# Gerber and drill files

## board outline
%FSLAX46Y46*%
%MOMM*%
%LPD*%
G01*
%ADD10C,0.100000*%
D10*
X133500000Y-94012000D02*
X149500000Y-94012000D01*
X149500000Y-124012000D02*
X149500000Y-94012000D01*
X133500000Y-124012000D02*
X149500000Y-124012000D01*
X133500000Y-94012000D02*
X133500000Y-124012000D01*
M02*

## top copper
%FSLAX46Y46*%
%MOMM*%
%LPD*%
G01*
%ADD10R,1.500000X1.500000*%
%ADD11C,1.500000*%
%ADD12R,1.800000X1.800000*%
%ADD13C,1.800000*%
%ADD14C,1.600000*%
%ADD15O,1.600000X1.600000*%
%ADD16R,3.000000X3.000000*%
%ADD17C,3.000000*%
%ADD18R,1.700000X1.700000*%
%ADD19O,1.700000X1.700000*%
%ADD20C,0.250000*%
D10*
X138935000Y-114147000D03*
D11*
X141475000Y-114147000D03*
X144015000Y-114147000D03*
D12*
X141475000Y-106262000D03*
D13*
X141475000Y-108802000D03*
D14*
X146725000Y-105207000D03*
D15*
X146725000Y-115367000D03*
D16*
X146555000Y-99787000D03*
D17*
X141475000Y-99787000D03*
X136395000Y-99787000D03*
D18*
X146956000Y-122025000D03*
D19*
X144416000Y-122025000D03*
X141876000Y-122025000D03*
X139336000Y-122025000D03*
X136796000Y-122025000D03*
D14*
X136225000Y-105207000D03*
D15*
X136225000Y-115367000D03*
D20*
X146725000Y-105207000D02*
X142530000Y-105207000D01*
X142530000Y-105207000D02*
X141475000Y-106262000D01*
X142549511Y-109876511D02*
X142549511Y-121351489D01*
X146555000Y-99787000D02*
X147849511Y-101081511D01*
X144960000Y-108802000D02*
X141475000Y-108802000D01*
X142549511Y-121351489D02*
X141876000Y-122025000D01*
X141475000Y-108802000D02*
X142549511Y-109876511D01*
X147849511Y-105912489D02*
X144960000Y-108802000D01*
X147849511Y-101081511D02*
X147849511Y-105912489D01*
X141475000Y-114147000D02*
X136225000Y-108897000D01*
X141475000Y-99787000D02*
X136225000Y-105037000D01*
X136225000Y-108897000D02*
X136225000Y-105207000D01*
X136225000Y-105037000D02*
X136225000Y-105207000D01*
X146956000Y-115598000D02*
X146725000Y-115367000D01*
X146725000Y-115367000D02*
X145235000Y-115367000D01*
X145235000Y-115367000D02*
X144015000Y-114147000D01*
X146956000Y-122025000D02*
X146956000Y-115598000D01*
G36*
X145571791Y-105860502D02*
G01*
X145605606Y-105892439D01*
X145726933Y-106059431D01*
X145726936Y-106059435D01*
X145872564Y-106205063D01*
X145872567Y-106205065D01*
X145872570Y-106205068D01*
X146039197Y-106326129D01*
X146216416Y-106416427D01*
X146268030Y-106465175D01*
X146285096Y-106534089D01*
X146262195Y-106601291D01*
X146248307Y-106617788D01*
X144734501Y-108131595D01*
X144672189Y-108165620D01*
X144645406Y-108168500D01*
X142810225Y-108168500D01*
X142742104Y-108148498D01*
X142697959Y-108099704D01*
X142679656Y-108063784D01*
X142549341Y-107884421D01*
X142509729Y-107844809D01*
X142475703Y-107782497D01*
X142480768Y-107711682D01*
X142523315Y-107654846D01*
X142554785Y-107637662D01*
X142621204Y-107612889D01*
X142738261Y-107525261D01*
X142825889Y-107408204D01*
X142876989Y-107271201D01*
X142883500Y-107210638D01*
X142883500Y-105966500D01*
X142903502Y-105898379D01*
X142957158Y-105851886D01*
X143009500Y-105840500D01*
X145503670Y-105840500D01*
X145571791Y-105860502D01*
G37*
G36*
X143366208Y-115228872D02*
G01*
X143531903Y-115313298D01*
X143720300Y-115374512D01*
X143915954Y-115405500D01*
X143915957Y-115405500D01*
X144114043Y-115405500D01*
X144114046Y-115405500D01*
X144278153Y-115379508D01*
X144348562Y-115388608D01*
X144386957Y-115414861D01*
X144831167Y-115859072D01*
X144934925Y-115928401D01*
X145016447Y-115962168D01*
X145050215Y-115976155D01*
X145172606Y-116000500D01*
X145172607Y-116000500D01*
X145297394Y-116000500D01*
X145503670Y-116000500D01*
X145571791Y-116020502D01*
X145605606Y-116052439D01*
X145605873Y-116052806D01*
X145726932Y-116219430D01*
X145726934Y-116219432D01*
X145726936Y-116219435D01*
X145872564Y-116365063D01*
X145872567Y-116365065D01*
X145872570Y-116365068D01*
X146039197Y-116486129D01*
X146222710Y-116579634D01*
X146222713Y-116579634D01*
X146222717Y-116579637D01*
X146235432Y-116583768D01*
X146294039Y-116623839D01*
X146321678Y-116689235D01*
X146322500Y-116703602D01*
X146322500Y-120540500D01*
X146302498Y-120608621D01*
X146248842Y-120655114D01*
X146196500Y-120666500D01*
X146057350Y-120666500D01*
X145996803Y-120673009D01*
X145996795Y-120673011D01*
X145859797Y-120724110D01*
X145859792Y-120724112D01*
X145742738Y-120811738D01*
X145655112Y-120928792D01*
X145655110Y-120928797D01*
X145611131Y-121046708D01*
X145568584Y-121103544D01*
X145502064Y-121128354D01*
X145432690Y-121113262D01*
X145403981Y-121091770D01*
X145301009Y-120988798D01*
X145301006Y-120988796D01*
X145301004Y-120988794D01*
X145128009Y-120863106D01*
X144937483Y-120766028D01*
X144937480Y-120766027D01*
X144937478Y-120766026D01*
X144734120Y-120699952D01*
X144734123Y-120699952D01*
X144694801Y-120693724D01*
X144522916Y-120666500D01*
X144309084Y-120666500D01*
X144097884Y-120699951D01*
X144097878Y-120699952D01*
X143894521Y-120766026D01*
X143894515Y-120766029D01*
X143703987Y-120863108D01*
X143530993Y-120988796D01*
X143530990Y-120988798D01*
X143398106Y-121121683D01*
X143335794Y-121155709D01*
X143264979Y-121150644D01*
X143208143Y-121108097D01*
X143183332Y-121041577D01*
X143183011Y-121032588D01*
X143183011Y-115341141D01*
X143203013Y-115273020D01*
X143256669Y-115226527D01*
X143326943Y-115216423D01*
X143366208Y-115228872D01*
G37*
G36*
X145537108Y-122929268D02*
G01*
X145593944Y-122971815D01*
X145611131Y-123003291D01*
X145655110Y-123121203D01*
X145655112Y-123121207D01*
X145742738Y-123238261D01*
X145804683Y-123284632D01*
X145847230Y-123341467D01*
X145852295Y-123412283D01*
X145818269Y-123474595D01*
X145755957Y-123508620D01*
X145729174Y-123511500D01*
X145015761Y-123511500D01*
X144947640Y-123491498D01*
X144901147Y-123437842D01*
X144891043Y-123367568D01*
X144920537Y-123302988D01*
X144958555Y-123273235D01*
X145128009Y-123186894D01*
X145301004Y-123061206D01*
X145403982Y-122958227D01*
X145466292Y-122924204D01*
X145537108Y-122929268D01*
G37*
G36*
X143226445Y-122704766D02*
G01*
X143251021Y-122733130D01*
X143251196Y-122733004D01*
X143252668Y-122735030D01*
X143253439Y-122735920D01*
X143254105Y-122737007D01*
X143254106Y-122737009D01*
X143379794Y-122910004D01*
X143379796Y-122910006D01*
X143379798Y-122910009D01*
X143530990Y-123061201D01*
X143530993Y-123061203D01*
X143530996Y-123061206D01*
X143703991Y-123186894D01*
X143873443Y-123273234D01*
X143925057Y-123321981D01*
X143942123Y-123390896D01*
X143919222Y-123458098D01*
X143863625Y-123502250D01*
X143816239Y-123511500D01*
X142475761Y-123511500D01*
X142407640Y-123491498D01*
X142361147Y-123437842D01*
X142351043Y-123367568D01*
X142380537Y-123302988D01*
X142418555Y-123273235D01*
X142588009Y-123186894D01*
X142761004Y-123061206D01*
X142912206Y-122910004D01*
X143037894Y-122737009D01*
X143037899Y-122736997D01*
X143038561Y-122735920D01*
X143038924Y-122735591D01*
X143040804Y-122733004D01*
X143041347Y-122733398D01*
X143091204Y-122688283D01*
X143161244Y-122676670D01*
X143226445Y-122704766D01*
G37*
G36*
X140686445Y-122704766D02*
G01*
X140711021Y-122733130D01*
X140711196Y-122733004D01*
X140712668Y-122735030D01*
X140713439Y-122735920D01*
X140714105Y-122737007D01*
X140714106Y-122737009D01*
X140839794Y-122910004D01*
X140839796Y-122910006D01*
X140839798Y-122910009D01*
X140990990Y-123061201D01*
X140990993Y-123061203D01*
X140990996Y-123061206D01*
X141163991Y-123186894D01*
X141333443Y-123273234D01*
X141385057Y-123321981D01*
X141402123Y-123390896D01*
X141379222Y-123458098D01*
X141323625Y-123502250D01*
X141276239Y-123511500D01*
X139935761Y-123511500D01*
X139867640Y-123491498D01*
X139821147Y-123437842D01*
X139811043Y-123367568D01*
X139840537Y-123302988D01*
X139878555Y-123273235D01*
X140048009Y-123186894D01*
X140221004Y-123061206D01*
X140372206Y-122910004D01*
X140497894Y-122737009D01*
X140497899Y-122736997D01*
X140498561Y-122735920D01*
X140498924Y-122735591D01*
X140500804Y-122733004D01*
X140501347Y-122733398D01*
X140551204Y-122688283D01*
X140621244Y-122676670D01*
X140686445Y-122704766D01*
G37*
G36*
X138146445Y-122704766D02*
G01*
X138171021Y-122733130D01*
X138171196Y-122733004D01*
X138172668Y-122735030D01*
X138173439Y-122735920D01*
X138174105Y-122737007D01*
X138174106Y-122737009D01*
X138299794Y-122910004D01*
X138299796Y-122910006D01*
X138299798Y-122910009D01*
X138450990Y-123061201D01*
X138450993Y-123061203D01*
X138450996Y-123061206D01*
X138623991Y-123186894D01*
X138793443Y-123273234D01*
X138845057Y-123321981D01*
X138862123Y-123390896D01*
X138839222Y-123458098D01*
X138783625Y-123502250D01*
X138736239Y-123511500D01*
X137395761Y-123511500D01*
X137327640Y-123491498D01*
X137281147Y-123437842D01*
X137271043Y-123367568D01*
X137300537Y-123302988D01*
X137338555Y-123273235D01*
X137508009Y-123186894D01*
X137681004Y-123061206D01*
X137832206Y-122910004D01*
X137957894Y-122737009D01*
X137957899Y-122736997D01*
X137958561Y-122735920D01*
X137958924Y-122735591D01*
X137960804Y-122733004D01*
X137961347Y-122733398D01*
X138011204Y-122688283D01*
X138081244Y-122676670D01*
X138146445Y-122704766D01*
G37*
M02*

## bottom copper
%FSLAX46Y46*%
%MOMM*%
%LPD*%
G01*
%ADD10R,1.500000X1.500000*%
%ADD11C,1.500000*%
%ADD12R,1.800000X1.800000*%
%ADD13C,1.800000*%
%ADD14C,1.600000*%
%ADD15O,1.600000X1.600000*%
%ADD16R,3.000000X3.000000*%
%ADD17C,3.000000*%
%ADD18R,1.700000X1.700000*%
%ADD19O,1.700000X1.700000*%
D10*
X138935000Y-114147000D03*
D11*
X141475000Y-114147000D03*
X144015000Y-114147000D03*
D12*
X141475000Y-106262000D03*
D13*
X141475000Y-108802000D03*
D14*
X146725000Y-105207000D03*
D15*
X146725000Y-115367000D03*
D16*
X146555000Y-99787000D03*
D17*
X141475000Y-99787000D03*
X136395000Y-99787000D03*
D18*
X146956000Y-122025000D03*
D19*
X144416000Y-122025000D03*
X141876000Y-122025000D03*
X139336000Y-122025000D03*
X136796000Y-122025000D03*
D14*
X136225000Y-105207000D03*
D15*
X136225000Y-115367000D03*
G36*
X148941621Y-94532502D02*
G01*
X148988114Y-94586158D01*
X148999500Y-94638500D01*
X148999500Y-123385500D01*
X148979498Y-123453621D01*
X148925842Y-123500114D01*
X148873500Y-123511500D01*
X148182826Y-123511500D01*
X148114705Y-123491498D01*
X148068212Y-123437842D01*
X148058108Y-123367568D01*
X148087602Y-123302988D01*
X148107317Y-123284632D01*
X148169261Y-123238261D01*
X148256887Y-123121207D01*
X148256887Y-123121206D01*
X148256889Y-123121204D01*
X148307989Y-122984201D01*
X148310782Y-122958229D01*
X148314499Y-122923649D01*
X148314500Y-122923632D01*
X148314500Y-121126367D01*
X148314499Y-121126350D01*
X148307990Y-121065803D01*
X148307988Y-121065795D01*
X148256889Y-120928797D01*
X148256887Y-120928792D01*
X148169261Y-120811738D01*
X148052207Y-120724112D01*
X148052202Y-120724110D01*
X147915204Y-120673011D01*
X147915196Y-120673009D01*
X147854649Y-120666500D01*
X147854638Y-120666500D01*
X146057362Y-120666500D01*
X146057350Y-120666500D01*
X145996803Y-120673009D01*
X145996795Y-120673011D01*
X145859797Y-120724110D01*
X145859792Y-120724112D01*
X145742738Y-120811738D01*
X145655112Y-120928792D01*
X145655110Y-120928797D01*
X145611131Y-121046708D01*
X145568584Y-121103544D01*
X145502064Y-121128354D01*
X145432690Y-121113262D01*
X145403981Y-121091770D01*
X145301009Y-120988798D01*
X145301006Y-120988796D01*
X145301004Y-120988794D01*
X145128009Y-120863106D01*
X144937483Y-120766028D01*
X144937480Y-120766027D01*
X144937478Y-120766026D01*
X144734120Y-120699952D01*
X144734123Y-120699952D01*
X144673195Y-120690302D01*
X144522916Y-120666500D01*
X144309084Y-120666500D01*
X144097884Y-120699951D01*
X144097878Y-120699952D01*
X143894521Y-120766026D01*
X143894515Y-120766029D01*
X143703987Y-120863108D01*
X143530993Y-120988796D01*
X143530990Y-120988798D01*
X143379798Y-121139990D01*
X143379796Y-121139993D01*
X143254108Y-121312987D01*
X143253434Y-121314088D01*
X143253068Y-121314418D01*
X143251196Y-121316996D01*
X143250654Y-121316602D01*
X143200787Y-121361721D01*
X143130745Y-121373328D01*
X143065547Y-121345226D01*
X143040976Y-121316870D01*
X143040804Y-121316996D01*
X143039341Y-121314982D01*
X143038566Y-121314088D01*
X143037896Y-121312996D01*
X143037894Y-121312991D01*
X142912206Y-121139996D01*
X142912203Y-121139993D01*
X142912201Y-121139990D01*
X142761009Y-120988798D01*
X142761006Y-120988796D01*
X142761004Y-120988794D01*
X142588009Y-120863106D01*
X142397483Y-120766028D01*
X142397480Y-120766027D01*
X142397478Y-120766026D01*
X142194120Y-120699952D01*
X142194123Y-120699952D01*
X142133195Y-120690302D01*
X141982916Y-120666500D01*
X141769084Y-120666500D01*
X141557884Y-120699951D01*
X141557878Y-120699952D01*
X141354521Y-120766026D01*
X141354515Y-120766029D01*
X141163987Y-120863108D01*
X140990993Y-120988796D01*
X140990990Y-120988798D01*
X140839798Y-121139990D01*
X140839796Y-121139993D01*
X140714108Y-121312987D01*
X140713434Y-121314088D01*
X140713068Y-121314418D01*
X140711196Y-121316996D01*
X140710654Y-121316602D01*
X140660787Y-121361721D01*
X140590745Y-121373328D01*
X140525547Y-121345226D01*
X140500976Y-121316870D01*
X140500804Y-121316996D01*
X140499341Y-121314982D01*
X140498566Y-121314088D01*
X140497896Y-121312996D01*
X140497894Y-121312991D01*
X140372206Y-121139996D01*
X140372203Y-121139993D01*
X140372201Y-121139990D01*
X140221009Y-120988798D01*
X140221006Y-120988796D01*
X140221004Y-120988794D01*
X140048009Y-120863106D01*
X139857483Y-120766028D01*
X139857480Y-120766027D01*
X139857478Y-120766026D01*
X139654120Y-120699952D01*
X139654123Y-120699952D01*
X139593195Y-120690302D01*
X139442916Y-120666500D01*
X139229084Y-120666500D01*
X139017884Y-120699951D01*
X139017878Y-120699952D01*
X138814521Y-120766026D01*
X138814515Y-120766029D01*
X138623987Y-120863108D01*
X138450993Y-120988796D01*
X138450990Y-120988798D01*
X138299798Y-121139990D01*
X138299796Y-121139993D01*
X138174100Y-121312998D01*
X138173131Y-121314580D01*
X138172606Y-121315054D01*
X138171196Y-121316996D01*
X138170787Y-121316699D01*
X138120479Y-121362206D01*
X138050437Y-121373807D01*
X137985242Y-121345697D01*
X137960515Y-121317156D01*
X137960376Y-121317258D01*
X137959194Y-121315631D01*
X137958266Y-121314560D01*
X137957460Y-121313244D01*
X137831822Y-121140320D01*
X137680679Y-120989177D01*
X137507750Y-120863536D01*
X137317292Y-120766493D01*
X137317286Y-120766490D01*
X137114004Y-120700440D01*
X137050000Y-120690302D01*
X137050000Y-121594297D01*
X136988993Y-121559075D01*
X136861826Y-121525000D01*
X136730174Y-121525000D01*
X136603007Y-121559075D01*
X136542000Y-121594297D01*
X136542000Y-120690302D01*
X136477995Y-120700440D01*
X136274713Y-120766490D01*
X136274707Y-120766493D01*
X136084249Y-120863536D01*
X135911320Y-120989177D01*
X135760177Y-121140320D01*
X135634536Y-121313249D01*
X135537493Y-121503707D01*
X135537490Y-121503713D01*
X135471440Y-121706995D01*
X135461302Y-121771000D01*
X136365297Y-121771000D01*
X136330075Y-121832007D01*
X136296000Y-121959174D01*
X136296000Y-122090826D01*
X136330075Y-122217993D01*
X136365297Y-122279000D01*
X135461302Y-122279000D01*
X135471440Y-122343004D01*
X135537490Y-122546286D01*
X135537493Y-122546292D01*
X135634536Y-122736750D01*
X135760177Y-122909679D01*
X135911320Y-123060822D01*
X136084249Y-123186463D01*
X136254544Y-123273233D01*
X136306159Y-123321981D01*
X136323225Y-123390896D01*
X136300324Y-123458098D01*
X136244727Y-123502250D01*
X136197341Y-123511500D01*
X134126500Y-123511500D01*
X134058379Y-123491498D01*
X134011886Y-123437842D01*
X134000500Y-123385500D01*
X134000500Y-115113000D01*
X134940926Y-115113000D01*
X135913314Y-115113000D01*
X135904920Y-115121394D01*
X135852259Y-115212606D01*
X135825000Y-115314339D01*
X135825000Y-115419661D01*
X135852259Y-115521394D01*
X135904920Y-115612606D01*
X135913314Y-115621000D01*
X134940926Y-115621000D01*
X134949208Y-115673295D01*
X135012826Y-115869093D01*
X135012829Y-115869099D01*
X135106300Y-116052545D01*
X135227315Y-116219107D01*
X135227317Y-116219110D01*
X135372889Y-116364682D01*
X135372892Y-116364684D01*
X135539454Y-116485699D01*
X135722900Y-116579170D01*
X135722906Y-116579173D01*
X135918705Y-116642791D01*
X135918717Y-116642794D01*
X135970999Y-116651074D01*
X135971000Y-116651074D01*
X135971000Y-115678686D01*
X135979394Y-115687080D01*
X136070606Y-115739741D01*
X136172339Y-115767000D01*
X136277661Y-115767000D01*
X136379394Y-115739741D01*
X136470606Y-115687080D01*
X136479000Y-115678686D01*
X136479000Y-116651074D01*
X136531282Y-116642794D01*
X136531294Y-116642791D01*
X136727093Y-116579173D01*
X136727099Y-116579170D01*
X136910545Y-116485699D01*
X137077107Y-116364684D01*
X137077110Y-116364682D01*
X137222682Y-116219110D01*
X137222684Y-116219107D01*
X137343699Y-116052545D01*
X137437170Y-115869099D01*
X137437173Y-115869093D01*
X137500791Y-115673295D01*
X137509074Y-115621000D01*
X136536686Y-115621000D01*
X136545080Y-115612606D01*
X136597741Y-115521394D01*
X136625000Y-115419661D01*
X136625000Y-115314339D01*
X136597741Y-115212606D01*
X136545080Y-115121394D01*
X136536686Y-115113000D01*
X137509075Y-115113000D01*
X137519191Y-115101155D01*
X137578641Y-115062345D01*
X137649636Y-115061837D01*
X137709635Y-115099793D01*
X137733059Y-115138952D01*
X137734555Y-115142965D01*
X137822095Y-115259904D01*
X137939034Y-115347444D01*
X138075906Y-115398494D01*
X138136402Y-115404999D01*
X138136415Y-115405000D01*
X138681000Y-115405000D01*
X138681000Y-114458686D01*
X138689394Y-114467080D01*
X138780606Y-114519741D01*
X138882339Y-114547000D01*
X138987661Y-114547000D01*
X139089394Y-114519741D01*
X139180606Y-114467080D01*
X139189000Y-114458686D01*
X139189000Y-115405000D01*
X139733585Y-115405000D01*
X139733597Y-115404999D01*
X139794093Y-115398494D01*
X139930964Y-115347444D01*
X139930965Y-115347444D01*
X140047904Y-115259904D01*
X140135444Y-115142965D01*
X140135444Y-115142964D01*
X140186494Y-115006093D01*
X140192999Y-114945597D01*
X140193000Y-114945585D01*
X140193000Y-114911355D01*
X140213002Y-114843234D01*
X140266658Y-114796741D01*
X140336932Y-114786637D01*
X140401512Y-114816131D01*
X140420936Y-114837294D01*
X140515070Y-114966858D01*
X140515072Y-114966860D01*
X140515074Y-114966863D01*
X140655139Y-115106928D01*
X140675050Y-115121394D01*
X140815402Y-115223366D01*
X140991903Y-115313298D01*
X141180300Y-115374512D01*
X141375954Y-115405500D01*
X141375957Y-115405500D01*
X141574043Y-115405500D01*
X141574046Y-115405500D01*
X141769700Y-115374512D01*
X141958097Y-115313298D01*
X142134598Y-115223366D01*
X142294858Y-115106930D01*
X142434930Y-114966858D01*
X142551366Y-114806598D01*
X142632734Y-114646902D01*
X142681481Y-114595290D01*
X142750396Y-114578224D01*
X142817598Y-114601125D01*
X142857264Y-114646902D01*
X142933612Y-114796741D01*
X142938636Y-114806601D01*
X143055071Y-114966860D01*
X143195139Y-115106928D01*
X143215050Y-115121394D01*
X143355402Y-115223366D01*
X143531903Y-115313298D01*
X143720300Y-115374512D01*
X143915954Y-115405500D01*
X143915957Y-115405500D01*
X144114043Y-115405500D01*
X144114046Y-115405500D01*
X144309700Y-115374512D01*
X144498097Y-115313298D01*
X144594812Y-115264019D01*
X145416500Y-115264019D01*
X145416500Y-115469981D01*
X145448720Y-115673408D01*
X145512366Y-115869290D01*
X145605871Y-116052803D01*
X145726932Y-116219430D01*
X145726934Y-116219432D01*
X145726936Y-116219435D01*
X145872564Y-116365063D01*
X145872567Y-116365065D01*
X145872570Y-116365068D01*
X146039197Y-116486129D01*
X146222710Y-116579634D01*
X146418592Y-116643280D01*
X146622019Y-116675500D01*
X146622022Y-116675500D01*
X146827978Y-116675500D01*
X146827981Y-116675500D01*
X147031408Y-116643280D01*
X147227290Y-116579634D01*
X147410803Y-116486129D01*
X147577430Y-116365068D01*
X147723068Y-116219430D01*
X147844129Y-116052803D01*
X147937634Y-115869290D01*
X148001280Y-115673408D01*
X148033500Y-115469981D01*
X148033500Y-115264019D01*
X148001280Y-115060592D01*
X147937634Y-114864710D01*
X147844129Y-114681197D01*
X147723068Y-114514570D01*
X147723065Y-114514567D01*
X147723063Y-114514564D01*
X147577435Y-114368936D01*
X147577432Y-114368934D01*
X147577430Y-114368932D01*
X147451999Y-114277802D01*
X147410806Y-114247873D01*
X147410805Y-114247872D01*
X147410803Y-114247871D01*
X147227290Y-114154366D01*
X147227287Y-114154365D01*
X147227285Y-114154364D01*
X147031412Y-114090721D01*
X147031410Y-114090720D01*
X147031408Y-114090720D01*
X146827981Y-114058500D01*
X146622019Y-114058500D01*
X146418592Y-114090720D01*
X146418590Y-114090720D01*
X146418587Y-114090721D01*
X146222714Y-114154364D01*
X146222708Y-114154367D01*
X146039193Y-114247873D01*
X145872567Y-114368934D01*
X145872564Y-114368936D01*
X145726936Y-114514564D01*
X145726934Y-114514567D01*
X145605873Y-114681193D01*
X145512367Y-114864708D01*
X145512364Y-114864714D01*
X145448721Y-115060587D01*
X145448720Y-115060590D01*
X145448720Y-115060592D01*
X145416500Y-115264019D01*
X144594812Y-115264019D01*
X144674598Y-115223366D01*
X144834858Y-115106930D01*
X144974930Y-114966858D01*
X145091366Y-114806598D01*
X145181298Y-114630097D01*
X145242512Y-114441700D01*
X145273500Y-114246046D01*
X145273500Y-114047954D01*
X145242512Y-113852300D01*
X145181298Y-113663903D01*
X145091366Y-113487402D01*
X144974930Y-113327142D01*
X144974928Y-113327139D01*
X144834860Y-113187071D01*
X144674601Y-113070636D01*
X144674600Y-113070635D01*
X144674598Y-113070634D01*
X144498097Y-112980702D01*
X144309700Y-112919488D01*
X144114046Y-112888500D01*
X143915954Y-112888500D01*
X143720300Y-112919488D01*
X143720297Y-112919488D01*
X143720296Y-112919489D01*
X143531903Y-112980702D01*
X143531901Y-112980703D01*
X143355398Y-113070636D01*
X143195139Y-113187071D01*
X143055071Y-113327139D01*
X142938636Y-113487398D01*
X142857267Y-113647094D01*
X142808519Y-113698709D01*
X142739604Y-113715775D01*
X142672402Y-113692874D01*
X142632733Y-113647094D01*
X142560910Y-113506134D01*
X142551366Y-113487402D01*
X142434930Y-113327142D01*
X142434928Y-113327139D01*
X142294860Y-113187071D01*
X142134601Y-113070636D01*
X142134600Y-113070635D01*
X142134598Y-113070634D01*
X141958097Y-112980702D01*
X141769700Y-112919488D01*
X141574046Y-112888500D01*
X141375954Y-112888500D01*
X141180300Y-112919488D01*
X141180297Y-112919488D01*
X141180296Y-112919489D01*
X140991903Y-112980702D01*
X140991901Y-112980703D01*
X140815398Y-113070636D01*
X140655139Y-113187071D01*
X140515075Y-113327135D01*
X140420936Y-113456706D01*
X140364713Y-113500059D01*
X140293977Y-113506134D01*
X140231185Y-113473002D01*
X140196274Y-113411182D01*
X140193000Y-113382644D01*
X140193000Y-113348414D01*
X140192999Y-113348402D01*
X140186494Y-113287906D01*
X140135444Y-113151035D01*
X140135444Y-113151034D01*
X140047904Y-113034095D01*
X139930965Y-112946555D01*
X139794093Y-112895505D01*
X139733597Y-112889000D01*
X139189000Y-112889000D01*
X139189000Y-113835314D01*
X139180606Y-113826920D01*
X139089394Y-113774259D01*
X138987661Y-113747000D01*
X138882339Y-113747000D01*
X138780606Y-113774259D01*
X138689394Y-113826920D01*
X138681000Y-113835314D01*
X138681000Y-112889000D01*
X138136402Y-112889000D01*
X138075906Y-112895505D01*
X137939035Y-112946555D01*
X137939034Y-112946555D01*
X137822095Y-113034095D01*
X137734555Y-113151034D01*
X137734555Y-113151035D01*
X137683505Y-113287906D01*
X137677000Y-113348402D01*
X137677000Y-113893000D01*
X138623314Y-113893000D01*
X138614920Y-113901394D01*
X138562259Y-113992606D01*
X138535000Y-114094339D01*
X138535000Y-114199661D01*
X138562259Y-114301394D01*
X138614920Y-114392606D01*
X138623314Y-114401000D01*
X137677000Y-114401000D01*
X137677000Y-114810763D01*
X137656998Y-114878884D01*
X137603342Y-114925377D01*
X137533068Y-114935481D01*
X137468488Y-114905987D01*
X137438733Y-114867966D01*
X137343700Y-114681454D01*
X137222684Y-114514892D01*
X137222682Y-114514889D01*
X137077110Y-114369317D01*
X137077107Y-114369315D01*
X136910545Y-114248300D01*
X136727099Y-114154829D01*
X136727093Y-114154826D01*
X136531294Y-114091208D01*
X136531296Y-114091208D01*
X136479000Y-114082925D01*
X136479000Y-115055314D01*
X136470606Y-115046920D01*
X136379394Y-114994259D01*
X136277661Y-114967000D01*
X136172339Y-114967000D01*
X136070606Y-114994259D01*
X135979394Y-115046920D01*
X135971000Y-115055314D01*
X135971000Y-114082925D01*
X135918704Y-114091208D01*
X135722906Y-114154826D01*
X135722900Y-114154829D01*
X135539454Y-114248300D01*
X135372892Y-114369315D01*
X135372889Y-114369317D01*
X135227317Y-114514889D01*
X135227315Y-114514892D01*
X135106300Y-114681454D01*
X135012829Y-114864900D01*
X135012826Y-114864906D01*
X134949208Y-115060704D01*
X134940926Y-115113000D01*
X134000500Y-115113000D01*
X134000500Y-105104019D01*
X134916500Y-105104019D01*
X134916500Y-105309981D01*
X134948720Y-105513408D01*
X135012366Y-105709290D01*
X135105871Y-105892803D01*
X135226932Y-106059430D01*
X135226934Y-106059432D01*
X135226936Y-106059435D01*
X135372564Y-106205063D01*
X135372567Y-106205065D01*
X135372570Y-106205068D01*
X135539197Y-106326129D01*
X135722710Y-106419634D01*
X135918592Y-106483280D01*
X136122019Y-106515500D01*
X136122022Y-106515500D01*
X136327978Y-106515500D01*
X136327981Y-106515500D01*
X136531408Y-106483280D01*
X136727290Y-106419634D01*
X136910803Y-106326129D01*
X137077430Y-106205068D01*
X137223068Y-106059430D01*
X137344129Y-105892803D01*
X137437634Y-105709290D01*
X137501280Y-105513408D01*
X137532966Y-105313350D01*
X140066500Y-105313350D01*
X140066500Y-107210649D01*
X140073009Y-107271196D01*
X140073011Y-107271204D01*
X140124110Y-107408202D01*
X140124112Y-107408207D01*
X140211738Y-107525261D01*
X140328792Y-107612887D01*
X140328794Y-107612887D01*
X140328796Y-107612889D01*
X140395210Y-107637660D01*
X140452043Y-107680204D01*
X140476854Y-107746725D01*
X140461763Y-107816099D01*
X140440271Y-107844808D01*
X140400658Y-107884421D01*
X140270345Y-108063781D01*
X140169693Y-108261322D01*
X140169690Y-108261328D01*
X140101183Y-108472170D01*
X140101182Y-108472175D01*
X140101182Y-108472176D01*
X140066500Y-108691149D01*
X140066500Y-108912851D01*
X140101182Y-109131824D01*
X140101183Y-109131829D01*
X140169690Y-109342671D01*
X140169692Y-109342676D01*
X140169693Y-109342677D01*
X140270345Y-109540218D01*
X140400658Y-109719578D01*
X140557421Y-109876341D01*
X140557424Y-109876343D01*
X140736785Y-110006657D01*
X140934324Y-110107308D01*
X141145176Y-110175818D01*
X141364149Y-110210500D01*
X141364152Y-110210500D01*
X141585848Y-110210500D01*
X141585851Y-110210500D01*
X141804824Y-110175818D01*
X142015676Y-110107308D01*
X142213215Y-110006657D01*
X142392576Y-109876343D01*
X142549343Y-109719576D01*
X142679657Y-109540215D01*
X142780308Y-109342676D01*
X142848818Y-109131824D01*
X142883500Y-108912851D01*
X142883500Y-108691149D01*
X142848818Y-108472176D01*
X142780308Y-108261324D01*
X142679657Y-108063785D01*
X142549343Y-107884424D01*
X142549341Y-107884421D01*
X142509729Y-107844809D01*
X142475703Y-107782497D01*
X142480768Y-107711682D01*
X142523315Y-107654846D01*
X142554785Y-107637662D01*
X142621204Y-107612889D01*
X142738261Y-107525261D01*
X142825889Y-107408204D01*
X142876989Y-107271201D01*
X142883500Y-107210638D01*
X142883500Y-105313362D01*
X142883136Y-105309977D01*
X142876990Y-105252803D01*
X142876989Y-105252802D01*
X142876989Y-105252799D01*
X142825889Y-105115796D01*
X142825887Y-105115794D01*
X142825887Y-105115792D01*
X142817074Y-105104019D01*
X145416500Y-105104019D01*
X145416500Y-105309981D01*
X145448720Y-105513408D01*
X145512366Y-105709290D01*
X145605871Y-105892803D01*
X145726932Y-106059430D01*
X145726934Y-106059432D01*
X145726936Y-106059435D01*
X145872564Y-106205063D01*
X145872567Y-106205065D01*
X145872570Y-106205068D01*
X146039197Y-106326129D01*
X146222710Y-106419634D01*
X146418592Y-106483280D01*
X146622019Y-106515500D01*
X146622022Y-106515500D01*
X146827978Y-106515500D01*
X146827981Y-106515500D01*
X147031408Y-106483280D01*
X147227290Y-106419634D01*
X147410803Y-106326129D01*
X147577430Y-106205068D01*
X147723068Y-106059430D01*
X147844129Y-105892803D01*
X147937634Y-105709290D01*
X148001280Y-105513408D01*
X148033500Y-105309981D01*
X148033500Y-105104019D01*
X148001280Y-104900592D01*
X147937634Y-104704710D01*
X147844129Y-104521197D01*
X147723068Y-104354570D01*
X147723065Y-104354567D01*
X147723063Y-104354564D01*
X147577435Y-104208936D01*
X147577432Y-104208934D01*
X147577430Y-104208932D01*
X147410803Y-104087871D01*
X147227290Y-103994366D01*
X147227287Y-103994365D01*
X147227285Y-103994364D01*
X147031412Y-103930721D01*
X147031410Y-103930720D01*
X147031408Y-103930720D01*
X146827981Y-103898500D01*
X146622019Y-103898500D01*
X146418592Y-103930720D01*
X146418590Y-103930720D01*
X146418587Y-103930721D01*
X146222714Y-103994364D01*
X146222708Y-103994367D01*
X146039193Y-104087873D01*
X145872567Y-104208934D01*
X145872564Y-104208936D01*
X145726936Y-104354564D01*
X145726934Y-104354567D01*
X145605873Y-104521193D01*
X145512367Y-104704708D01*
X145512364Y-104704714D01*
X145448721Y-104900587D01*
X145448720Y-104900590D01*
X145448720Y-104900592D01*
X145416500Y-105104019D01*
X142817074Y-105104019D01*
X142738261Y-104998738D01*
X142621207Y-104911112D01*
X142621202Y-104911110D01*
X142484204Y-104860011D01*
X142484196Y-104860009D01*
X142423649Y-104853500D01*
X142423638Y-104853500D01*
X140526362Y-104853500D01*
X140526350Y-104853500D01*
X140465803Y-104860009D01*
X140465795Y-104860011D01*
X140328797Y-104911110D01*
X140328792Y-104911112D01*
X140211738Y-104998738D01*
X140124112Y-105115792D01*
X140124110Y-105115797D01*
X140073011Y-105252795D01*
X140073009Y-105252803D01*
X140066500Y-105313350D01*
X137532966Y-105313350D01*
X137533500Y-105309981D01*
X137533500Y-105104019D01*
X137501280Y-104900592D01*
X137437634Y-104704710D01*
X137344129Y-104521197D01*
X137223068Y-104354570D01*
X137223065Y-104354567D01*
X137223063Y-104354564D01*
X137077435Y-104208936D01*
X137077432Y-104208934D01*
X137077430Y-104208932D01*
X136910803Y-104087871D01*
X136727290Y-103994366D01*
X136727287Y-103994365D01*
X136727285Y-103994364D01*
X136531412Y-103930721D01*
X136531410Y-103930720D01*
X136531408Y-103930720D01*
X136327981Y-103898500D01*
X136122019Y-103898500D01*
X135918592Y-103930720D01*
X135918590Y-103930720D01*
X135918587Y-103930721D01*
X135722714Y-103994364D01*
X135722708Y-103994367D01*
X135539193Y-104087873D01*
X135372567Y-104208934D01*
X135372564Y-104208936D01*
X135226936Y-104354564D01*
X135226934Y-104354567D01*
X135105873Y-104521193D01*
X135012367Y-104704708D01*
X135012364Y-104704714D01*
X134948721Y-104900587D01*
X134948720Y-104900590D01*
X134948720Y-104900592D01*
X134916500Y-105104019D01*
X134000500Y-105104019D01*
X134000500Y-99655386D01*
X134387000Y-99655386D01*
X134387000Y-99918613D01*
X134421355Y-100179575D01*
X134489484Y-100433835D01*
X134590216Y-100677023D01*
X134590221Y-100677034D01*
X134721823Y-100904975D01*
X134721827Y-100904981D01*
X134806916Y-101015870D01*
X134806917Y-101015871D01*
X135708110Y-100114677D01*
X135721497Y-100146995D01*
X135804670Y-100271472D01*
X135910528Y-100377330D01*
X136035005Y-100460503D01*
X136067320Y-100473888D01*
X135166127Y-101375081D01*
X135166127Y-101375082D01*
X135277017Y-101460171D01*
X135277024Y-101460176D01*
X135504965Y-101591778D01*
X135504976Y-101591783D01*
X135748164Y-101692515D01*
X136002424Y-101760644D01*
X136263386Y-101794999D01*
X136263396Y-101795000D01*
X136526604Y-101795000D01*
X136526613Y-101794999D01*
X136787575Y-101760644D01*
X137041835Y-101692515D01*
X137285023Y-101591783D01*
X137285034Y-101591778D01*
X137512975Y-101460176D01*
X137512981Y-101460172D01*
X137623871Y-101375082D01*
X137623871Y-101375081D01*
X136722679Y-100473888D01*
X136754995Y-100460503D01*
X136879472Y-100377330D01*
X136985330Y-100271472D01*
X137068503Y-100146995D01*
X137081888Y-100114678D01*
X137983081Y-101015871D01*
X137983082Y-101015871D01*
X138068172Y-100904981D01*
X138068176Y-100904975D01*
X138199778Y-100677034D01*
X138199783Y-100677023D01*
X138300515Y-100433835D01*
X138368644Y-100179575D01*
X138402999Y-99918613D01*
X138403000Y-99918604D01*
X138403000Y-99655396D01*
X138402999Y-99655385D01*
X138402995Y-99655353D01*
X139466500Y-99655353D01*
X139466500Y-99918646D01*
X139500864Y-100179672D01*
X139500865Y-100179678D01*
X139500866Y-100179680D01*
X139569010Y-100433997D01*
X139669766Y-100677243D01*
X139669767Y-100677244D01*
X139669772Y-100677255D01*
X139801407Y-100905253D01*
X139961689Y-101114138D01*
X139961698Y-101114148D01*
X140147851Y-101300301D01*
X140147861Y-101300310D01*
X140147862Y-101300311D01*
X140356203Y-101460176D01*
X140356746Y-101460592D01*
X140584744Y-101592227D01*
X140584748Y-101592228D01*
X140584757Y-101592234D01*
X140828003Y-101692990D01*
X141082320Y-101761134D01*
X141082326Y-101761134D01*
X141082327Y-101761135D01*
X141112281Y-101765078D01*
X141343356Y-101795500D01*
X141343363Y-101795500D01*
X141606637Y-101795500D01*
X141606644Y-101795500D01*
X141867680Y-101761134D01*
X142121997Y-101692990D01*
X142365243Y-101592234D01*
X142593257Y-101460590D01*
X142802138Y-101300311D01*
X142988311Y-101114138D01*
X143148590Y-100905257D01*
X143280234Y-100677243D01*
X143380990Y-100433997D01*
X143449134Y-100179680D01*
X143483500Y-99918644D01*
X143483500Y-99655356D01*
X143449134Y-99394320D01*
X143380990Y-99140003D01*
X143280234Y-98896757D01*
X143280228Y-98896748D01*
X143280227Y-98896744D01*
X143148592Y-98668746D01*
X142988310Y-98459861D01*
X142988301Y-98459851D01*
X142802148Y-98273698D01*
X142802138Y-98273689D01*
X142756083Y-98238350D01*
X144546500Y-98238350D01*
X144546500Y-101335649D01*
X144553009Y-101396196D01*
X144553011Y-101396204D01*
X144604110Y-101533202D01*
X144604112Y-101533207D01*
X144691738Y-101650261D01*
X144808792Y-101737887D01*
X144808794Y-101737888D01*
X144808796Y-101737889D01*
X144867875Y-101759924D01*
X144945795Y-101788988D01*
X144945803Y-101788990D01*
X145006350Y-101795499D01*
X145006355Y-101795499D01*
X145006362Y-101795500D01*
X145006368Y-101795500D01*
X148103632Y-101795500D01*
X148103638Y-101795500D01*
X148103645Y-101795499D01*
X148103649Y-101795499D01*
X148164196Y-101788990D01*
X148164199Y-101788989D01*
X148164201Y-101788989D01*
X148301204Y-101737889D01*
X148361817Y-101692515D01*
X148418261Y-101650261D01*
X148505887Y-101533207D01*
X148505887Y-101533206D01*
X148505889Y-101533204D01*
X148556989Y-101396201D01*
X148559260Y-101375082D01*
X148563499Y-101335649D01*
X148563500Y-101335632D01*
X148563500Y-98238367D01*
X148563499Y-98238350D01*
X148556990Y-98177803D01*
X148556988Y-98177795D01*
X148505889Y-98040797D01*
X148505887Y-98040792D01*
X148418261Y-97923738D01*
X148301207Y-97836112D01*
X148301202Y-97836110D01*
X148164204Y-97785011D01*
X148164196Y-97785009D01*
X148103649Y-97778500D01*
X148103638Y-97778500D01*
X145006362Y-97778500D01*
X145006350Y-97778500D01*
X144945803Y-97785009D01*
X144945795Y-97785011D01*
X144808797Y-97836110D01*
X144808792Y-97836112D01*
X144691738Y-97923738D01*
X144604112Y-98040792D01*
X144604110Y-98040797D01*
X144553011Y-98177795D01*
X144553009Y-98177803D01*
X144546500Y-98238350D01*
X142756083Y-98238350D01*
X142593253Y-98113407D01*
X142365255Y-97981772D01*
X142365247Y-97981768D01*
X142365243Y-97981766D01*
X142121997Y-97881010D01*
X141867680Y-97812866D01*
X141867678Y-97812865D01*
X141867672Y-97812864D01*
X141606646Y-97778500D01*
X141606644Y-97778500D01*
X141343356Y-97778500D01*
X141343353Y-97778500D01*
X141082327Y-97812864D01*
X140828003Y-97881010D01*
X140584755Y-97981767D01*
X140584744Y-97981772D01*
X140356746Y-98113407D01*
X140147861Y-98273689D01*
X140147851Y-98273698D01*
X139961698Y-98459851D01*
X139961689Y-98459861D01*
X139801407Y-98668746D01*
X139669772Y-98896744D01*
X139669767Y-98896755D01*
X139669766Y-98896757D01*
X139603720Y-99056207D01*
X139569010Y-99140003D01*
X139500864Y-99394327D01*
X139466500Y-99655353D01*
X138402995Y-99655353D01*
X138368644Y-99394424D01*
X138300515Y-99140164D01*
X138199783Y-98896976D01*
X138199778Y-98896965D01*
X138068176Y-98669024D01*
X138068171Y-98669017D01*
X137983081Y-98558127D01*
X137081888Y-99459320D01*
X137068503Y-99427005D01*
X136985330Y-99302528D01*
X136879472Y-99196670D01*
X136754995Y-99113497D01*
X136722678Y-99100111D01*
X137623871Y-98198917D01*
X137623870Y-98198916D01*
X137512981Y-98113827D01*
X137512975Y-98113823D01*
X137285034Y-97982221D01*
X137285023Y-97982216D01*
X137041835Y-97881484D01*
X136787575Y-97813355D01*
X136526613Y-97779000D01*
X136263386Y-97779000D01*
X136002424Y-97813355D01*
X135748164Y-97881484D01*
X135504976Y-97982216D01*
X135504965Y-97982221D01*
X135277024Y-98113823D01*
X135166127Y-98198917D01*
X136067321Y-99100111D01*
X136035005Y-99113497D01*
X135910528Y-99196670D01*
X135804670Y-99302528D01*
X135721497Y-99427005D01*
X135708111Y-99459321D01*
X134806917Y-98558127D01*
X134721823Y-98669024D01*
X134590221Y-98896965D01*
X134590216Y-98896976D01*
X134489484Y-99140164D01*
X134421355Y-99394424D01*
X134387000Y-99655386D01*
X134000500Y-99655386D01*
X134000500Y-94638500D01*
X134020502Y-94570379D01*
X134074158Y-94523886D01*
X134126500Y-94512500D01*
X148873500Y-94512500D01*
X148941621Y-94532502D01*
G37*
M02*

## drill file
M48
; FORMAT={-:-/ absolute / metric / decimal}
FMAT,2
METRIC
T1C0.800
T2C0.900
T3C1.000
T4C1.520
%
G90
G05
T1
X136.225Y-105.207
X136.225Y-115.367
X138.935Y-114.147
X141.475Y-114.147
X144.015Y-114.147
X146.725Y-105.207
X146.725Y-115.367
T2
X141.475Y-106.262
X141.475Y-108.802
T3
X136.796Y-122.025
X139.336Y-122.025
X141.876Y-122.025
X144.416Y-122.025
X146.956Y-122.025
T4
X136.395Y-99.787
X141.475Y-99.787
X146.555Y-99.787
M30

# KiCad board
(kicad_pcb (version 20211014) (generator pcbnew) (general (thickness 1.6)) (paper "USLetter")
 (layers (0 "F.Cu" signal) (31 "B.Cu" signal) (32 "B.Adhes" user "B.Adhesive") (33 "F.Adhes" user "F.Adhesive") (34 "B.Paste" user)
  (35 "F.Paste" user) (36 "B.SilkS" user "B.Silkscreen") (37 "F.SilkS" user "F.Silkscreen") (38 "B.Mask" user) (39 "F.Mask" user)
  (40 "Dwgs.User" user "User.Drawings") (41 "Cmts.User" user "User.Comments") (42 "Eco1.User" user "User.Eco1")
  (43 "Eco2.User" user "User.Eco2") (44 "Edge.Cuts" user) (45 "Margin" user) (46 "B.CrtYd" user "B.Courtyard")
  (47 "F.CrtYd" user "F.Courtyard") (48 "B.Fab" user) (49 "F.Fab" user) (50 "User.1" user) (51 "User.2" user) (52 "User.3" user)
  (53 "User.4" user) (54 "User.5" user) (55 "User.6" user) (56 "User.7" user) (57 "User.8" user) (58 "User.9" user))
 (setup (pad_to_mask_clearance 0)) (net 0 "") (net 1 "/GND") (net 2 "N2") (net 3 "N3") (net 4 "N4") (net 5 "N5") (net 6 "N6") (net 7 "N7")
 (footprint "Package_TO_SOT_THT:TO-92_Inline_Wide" (layer "F.Cu") (at 138.935 114.147)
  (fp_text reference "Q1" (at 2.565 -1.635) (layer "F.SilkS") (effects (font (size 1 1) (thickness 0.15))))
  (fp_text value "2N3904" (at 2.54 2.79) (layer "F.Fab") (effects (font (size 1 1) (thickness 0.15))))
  (pad "1" thru_hole rect locked (at 0 0) (size 1.5 1.5) (drill 0.8) (layers *.Cu *.Mask) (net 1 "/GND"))
  (pad "2" thru_hole circle locked (at 2.54 0) (size 1.5 1.5) (drill 0.8) (layers *.Cu *.Mask) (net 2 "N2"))
  (pad "3" thru_hole circle locked (at 5.08 0) (size 1.5 1.5) (drill 0.8) (layers *.Cu *.Mask) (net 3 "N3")))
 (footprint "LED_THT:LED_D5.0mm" (layer "F.Cu") (at 141.475 106.262 -90)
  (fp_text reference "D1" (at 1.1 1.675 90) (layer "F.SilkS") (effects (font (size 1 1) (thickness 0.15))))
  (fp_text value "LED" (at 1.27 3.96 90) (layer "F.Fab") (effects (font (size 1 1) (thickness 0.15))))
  (pad "1" thru_hole rect locked (at 0 0 270) (size 1.8 1.8) (drill 0.9) (layers *.Cu *.Mask) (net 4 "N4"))
  (pad "2" thru_hole circle locked (at 2.54 0 270) (size 1.8 1.8) (drill 0.9) (layers *.Cu *.Mask) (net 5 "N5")))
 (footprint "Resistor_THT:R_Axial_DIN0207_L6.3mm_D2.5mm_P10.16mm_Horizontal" (layer "F.Cu") (at 146.725 105.207 -90)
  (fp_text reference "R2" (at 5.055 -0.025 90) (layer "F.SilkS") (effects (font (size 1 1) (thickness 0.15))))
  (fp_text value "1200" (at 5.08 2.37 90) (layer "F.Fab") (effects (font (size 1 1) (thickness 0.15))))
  (pad "1" thru_hole circle locked (at 0 0 270) (size 1.6 1.6) (drill 0.8) (layers *.Cu *.Mask) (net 4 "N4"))
  (pad "2" thru_hole oval locked (at 10.16 0 270) (size 1.6 1.6) (drill 0.8) (layers *.Cu *.Mask) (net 3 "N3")))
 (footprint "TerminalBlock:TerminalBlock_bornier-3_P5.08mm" (layer "F.Cu") (at 146.555 99.787 180)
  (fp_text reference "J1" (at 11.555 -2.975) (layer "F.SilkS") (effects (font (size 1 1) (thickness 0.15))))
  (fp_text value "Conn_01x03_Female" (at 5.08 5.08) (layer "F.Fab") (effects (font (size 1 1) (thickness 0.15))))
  (pad "1" thru_hole rect locked (at 0 0 180) (size 3 3) (drill 1.52) (layers *.Cu *.Mask) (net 5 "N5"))
  (pad "2" thru_hole circle locked (at 5.08 0 180) (size 3 3) (drill 1.52) (layers *.Cu *.Mask) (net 2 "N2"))
  (pad "3" thru_hole circle locked (at 10.16 0 180) (size 3 3) (drill 1.52) (layers *.Cu *.Mask) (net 1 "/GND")))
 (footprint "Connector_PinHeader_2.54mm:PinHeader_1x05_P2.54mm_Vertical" (layer "F.Cu") (at 146.956 122.025 -90)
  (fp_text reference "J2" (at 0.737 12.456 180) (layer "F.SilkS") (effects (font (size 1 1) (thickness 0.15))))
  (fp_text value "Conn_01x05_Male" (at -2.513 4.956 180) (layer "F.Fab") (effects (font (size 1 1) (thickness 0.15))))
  (pad "1" thru_hole rect locked (at 0 0 270) (size 1.7 1.7) (drill 1) (layers *.Cu *.Mask) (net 3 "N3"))
  (pad "2" thru_hole oval locked (at 0 2.54 270) (size 1.7 1.7) (drill 1) (layers *.Cu *.Mask) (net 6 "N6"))
  (pad "3" thru_hole oval locked (at 0 5.08 270) (size 1.7 1.7) (drill 1) (layers *.Cu *.Mask) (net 5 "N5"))
  (pad "4" thru_hole oval locked (at 0 7.62 270) (size 1.7 1.7) (drill 1) (layers *.Cu *.Mask) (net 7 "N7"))
  (pad "5" thru_hole oval locked (at 0 10.16 270) (size 1.7 1.7) (drill 1) (layers *.Cu *.Mask) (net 1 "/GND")))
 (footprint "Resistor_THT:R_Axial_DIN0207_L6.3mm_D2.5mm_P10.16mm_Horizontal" (layer "F.Cu") (at 136.225 105.207 -90)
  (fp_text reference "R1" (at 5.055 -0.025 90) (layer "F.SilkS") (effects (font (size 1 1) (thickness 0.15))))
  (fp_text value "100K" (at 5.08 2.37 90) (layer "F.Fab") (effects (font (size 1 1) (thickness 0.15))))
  (pad "1" thru_hole circle locked (at 0 0 270) (size 1.6 1.6) (drill 0.8) (layers *.Cu *.Mask) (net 2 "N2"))
  (pad "2" thru_hole oval locked (at 10.16 0 270) (size 1.6 1.6) (drill 0.8) (layers *.Cu *.Mask) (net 1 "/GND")))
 (gr_line (start 133.5 94.012) (end 149.5 94.012) (layer "Edge.Cuts") (width 0.1))
 (gr_line (start 149.5 124.012) (end 149.5 94.012) (layer "Edge.Cuts") (width 0.1))
 (gr_line (start 133.5 124.012) (end 149.5 124.012) (layer "Edge.Cuts") (width 0.1))
 (gr_line (start 133.5 94.012) (end 133.5 124.012) (layer "Edge.Cuts") (width 0.1))
 (segment (start 146.725 105.207) (end 142.53 105.207) (width 0.25) (layer "F.Cu") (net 4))
 (segment (start 142.53 105.207) (end 141.475 106.262) (width 0.25) (layer "F.Cu") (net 4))
 (segment (start 142.549511 109.876511) (end 142.549511 121.351489) (width 0.25) (layer "F.Cu") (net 5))
 (segment (start 146.555 99.787) (end 147.849511 101.081511) (width 0.25) (layer "F.Cu") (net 5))
 (segment (start 144.96 108.802) (end 141.475 108.802) (width 0.25) (layer "F.Cu") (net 5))
 (segment (start 142.549511 121.351489) (end 141.876 122.025) (width 0.25) (layer "F.Cu") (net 5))
 (segment (start 141.475 108.802) (end 142.549511 109.876511) (width 0.25) (layer "F.Cu") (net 5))
 (segment (start 147.849511 105.912489) (end 144.96 108.802) (width 0.25) (layer "F.Cu") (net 5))
 (segment (start 147.849511 101.081511) (end 147.849511 105.912489) (width 0.25) (layer "F.Cu") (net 5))
 (segment (start 141.475 114.147) (end 136.225 108.897) (width 0.25) (layer "F.Cu") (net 2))
 (segment (start 141.475 99.787) (end 136.225 105.037) (width 0.25) (layer "F.Cu") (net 2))
 (segment (start 136.225 108.897) (end 136.225 105.207) (width 0.25) (layer "F.Cu") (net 2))
 (segment (start 136.225 105.037) (end 136.225 105.207) (width 0.25) (layer "F.Cu") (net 2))
 (segment (start 146.956 115.598) (end 146.725 115.367) (width 0.25) (layer "F.Cu") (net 3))
 (segment (start 146.725 115.367) (end 145.235 115.367) (width 0.25) (layer "F.Cu") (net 3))
 (segment (start 145.235 115.367) (end 144.015 114.147) (width 0.25) (layer "F.Cu") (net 3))
 (segment (start 146.956 122.025) (end 146.956 115.598) (width 0.25) (layer "F.Cu") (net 3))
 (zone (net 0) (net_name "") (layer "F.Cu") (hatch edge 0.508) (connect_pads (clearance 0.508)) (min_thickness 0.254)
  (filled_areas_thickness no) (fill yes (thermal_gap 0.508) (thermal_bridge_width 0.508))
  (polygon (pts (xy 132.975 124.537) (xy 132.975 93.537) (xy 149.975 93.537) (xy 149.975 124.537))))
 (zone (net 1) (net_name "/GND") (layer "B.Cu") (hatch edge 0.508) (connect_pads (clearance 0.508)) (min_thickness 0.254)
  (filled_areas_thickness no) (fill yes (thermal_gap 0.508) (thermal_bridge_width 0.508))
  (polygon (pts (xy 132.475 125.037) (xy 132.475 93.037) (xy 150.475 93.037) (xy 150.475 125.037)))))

